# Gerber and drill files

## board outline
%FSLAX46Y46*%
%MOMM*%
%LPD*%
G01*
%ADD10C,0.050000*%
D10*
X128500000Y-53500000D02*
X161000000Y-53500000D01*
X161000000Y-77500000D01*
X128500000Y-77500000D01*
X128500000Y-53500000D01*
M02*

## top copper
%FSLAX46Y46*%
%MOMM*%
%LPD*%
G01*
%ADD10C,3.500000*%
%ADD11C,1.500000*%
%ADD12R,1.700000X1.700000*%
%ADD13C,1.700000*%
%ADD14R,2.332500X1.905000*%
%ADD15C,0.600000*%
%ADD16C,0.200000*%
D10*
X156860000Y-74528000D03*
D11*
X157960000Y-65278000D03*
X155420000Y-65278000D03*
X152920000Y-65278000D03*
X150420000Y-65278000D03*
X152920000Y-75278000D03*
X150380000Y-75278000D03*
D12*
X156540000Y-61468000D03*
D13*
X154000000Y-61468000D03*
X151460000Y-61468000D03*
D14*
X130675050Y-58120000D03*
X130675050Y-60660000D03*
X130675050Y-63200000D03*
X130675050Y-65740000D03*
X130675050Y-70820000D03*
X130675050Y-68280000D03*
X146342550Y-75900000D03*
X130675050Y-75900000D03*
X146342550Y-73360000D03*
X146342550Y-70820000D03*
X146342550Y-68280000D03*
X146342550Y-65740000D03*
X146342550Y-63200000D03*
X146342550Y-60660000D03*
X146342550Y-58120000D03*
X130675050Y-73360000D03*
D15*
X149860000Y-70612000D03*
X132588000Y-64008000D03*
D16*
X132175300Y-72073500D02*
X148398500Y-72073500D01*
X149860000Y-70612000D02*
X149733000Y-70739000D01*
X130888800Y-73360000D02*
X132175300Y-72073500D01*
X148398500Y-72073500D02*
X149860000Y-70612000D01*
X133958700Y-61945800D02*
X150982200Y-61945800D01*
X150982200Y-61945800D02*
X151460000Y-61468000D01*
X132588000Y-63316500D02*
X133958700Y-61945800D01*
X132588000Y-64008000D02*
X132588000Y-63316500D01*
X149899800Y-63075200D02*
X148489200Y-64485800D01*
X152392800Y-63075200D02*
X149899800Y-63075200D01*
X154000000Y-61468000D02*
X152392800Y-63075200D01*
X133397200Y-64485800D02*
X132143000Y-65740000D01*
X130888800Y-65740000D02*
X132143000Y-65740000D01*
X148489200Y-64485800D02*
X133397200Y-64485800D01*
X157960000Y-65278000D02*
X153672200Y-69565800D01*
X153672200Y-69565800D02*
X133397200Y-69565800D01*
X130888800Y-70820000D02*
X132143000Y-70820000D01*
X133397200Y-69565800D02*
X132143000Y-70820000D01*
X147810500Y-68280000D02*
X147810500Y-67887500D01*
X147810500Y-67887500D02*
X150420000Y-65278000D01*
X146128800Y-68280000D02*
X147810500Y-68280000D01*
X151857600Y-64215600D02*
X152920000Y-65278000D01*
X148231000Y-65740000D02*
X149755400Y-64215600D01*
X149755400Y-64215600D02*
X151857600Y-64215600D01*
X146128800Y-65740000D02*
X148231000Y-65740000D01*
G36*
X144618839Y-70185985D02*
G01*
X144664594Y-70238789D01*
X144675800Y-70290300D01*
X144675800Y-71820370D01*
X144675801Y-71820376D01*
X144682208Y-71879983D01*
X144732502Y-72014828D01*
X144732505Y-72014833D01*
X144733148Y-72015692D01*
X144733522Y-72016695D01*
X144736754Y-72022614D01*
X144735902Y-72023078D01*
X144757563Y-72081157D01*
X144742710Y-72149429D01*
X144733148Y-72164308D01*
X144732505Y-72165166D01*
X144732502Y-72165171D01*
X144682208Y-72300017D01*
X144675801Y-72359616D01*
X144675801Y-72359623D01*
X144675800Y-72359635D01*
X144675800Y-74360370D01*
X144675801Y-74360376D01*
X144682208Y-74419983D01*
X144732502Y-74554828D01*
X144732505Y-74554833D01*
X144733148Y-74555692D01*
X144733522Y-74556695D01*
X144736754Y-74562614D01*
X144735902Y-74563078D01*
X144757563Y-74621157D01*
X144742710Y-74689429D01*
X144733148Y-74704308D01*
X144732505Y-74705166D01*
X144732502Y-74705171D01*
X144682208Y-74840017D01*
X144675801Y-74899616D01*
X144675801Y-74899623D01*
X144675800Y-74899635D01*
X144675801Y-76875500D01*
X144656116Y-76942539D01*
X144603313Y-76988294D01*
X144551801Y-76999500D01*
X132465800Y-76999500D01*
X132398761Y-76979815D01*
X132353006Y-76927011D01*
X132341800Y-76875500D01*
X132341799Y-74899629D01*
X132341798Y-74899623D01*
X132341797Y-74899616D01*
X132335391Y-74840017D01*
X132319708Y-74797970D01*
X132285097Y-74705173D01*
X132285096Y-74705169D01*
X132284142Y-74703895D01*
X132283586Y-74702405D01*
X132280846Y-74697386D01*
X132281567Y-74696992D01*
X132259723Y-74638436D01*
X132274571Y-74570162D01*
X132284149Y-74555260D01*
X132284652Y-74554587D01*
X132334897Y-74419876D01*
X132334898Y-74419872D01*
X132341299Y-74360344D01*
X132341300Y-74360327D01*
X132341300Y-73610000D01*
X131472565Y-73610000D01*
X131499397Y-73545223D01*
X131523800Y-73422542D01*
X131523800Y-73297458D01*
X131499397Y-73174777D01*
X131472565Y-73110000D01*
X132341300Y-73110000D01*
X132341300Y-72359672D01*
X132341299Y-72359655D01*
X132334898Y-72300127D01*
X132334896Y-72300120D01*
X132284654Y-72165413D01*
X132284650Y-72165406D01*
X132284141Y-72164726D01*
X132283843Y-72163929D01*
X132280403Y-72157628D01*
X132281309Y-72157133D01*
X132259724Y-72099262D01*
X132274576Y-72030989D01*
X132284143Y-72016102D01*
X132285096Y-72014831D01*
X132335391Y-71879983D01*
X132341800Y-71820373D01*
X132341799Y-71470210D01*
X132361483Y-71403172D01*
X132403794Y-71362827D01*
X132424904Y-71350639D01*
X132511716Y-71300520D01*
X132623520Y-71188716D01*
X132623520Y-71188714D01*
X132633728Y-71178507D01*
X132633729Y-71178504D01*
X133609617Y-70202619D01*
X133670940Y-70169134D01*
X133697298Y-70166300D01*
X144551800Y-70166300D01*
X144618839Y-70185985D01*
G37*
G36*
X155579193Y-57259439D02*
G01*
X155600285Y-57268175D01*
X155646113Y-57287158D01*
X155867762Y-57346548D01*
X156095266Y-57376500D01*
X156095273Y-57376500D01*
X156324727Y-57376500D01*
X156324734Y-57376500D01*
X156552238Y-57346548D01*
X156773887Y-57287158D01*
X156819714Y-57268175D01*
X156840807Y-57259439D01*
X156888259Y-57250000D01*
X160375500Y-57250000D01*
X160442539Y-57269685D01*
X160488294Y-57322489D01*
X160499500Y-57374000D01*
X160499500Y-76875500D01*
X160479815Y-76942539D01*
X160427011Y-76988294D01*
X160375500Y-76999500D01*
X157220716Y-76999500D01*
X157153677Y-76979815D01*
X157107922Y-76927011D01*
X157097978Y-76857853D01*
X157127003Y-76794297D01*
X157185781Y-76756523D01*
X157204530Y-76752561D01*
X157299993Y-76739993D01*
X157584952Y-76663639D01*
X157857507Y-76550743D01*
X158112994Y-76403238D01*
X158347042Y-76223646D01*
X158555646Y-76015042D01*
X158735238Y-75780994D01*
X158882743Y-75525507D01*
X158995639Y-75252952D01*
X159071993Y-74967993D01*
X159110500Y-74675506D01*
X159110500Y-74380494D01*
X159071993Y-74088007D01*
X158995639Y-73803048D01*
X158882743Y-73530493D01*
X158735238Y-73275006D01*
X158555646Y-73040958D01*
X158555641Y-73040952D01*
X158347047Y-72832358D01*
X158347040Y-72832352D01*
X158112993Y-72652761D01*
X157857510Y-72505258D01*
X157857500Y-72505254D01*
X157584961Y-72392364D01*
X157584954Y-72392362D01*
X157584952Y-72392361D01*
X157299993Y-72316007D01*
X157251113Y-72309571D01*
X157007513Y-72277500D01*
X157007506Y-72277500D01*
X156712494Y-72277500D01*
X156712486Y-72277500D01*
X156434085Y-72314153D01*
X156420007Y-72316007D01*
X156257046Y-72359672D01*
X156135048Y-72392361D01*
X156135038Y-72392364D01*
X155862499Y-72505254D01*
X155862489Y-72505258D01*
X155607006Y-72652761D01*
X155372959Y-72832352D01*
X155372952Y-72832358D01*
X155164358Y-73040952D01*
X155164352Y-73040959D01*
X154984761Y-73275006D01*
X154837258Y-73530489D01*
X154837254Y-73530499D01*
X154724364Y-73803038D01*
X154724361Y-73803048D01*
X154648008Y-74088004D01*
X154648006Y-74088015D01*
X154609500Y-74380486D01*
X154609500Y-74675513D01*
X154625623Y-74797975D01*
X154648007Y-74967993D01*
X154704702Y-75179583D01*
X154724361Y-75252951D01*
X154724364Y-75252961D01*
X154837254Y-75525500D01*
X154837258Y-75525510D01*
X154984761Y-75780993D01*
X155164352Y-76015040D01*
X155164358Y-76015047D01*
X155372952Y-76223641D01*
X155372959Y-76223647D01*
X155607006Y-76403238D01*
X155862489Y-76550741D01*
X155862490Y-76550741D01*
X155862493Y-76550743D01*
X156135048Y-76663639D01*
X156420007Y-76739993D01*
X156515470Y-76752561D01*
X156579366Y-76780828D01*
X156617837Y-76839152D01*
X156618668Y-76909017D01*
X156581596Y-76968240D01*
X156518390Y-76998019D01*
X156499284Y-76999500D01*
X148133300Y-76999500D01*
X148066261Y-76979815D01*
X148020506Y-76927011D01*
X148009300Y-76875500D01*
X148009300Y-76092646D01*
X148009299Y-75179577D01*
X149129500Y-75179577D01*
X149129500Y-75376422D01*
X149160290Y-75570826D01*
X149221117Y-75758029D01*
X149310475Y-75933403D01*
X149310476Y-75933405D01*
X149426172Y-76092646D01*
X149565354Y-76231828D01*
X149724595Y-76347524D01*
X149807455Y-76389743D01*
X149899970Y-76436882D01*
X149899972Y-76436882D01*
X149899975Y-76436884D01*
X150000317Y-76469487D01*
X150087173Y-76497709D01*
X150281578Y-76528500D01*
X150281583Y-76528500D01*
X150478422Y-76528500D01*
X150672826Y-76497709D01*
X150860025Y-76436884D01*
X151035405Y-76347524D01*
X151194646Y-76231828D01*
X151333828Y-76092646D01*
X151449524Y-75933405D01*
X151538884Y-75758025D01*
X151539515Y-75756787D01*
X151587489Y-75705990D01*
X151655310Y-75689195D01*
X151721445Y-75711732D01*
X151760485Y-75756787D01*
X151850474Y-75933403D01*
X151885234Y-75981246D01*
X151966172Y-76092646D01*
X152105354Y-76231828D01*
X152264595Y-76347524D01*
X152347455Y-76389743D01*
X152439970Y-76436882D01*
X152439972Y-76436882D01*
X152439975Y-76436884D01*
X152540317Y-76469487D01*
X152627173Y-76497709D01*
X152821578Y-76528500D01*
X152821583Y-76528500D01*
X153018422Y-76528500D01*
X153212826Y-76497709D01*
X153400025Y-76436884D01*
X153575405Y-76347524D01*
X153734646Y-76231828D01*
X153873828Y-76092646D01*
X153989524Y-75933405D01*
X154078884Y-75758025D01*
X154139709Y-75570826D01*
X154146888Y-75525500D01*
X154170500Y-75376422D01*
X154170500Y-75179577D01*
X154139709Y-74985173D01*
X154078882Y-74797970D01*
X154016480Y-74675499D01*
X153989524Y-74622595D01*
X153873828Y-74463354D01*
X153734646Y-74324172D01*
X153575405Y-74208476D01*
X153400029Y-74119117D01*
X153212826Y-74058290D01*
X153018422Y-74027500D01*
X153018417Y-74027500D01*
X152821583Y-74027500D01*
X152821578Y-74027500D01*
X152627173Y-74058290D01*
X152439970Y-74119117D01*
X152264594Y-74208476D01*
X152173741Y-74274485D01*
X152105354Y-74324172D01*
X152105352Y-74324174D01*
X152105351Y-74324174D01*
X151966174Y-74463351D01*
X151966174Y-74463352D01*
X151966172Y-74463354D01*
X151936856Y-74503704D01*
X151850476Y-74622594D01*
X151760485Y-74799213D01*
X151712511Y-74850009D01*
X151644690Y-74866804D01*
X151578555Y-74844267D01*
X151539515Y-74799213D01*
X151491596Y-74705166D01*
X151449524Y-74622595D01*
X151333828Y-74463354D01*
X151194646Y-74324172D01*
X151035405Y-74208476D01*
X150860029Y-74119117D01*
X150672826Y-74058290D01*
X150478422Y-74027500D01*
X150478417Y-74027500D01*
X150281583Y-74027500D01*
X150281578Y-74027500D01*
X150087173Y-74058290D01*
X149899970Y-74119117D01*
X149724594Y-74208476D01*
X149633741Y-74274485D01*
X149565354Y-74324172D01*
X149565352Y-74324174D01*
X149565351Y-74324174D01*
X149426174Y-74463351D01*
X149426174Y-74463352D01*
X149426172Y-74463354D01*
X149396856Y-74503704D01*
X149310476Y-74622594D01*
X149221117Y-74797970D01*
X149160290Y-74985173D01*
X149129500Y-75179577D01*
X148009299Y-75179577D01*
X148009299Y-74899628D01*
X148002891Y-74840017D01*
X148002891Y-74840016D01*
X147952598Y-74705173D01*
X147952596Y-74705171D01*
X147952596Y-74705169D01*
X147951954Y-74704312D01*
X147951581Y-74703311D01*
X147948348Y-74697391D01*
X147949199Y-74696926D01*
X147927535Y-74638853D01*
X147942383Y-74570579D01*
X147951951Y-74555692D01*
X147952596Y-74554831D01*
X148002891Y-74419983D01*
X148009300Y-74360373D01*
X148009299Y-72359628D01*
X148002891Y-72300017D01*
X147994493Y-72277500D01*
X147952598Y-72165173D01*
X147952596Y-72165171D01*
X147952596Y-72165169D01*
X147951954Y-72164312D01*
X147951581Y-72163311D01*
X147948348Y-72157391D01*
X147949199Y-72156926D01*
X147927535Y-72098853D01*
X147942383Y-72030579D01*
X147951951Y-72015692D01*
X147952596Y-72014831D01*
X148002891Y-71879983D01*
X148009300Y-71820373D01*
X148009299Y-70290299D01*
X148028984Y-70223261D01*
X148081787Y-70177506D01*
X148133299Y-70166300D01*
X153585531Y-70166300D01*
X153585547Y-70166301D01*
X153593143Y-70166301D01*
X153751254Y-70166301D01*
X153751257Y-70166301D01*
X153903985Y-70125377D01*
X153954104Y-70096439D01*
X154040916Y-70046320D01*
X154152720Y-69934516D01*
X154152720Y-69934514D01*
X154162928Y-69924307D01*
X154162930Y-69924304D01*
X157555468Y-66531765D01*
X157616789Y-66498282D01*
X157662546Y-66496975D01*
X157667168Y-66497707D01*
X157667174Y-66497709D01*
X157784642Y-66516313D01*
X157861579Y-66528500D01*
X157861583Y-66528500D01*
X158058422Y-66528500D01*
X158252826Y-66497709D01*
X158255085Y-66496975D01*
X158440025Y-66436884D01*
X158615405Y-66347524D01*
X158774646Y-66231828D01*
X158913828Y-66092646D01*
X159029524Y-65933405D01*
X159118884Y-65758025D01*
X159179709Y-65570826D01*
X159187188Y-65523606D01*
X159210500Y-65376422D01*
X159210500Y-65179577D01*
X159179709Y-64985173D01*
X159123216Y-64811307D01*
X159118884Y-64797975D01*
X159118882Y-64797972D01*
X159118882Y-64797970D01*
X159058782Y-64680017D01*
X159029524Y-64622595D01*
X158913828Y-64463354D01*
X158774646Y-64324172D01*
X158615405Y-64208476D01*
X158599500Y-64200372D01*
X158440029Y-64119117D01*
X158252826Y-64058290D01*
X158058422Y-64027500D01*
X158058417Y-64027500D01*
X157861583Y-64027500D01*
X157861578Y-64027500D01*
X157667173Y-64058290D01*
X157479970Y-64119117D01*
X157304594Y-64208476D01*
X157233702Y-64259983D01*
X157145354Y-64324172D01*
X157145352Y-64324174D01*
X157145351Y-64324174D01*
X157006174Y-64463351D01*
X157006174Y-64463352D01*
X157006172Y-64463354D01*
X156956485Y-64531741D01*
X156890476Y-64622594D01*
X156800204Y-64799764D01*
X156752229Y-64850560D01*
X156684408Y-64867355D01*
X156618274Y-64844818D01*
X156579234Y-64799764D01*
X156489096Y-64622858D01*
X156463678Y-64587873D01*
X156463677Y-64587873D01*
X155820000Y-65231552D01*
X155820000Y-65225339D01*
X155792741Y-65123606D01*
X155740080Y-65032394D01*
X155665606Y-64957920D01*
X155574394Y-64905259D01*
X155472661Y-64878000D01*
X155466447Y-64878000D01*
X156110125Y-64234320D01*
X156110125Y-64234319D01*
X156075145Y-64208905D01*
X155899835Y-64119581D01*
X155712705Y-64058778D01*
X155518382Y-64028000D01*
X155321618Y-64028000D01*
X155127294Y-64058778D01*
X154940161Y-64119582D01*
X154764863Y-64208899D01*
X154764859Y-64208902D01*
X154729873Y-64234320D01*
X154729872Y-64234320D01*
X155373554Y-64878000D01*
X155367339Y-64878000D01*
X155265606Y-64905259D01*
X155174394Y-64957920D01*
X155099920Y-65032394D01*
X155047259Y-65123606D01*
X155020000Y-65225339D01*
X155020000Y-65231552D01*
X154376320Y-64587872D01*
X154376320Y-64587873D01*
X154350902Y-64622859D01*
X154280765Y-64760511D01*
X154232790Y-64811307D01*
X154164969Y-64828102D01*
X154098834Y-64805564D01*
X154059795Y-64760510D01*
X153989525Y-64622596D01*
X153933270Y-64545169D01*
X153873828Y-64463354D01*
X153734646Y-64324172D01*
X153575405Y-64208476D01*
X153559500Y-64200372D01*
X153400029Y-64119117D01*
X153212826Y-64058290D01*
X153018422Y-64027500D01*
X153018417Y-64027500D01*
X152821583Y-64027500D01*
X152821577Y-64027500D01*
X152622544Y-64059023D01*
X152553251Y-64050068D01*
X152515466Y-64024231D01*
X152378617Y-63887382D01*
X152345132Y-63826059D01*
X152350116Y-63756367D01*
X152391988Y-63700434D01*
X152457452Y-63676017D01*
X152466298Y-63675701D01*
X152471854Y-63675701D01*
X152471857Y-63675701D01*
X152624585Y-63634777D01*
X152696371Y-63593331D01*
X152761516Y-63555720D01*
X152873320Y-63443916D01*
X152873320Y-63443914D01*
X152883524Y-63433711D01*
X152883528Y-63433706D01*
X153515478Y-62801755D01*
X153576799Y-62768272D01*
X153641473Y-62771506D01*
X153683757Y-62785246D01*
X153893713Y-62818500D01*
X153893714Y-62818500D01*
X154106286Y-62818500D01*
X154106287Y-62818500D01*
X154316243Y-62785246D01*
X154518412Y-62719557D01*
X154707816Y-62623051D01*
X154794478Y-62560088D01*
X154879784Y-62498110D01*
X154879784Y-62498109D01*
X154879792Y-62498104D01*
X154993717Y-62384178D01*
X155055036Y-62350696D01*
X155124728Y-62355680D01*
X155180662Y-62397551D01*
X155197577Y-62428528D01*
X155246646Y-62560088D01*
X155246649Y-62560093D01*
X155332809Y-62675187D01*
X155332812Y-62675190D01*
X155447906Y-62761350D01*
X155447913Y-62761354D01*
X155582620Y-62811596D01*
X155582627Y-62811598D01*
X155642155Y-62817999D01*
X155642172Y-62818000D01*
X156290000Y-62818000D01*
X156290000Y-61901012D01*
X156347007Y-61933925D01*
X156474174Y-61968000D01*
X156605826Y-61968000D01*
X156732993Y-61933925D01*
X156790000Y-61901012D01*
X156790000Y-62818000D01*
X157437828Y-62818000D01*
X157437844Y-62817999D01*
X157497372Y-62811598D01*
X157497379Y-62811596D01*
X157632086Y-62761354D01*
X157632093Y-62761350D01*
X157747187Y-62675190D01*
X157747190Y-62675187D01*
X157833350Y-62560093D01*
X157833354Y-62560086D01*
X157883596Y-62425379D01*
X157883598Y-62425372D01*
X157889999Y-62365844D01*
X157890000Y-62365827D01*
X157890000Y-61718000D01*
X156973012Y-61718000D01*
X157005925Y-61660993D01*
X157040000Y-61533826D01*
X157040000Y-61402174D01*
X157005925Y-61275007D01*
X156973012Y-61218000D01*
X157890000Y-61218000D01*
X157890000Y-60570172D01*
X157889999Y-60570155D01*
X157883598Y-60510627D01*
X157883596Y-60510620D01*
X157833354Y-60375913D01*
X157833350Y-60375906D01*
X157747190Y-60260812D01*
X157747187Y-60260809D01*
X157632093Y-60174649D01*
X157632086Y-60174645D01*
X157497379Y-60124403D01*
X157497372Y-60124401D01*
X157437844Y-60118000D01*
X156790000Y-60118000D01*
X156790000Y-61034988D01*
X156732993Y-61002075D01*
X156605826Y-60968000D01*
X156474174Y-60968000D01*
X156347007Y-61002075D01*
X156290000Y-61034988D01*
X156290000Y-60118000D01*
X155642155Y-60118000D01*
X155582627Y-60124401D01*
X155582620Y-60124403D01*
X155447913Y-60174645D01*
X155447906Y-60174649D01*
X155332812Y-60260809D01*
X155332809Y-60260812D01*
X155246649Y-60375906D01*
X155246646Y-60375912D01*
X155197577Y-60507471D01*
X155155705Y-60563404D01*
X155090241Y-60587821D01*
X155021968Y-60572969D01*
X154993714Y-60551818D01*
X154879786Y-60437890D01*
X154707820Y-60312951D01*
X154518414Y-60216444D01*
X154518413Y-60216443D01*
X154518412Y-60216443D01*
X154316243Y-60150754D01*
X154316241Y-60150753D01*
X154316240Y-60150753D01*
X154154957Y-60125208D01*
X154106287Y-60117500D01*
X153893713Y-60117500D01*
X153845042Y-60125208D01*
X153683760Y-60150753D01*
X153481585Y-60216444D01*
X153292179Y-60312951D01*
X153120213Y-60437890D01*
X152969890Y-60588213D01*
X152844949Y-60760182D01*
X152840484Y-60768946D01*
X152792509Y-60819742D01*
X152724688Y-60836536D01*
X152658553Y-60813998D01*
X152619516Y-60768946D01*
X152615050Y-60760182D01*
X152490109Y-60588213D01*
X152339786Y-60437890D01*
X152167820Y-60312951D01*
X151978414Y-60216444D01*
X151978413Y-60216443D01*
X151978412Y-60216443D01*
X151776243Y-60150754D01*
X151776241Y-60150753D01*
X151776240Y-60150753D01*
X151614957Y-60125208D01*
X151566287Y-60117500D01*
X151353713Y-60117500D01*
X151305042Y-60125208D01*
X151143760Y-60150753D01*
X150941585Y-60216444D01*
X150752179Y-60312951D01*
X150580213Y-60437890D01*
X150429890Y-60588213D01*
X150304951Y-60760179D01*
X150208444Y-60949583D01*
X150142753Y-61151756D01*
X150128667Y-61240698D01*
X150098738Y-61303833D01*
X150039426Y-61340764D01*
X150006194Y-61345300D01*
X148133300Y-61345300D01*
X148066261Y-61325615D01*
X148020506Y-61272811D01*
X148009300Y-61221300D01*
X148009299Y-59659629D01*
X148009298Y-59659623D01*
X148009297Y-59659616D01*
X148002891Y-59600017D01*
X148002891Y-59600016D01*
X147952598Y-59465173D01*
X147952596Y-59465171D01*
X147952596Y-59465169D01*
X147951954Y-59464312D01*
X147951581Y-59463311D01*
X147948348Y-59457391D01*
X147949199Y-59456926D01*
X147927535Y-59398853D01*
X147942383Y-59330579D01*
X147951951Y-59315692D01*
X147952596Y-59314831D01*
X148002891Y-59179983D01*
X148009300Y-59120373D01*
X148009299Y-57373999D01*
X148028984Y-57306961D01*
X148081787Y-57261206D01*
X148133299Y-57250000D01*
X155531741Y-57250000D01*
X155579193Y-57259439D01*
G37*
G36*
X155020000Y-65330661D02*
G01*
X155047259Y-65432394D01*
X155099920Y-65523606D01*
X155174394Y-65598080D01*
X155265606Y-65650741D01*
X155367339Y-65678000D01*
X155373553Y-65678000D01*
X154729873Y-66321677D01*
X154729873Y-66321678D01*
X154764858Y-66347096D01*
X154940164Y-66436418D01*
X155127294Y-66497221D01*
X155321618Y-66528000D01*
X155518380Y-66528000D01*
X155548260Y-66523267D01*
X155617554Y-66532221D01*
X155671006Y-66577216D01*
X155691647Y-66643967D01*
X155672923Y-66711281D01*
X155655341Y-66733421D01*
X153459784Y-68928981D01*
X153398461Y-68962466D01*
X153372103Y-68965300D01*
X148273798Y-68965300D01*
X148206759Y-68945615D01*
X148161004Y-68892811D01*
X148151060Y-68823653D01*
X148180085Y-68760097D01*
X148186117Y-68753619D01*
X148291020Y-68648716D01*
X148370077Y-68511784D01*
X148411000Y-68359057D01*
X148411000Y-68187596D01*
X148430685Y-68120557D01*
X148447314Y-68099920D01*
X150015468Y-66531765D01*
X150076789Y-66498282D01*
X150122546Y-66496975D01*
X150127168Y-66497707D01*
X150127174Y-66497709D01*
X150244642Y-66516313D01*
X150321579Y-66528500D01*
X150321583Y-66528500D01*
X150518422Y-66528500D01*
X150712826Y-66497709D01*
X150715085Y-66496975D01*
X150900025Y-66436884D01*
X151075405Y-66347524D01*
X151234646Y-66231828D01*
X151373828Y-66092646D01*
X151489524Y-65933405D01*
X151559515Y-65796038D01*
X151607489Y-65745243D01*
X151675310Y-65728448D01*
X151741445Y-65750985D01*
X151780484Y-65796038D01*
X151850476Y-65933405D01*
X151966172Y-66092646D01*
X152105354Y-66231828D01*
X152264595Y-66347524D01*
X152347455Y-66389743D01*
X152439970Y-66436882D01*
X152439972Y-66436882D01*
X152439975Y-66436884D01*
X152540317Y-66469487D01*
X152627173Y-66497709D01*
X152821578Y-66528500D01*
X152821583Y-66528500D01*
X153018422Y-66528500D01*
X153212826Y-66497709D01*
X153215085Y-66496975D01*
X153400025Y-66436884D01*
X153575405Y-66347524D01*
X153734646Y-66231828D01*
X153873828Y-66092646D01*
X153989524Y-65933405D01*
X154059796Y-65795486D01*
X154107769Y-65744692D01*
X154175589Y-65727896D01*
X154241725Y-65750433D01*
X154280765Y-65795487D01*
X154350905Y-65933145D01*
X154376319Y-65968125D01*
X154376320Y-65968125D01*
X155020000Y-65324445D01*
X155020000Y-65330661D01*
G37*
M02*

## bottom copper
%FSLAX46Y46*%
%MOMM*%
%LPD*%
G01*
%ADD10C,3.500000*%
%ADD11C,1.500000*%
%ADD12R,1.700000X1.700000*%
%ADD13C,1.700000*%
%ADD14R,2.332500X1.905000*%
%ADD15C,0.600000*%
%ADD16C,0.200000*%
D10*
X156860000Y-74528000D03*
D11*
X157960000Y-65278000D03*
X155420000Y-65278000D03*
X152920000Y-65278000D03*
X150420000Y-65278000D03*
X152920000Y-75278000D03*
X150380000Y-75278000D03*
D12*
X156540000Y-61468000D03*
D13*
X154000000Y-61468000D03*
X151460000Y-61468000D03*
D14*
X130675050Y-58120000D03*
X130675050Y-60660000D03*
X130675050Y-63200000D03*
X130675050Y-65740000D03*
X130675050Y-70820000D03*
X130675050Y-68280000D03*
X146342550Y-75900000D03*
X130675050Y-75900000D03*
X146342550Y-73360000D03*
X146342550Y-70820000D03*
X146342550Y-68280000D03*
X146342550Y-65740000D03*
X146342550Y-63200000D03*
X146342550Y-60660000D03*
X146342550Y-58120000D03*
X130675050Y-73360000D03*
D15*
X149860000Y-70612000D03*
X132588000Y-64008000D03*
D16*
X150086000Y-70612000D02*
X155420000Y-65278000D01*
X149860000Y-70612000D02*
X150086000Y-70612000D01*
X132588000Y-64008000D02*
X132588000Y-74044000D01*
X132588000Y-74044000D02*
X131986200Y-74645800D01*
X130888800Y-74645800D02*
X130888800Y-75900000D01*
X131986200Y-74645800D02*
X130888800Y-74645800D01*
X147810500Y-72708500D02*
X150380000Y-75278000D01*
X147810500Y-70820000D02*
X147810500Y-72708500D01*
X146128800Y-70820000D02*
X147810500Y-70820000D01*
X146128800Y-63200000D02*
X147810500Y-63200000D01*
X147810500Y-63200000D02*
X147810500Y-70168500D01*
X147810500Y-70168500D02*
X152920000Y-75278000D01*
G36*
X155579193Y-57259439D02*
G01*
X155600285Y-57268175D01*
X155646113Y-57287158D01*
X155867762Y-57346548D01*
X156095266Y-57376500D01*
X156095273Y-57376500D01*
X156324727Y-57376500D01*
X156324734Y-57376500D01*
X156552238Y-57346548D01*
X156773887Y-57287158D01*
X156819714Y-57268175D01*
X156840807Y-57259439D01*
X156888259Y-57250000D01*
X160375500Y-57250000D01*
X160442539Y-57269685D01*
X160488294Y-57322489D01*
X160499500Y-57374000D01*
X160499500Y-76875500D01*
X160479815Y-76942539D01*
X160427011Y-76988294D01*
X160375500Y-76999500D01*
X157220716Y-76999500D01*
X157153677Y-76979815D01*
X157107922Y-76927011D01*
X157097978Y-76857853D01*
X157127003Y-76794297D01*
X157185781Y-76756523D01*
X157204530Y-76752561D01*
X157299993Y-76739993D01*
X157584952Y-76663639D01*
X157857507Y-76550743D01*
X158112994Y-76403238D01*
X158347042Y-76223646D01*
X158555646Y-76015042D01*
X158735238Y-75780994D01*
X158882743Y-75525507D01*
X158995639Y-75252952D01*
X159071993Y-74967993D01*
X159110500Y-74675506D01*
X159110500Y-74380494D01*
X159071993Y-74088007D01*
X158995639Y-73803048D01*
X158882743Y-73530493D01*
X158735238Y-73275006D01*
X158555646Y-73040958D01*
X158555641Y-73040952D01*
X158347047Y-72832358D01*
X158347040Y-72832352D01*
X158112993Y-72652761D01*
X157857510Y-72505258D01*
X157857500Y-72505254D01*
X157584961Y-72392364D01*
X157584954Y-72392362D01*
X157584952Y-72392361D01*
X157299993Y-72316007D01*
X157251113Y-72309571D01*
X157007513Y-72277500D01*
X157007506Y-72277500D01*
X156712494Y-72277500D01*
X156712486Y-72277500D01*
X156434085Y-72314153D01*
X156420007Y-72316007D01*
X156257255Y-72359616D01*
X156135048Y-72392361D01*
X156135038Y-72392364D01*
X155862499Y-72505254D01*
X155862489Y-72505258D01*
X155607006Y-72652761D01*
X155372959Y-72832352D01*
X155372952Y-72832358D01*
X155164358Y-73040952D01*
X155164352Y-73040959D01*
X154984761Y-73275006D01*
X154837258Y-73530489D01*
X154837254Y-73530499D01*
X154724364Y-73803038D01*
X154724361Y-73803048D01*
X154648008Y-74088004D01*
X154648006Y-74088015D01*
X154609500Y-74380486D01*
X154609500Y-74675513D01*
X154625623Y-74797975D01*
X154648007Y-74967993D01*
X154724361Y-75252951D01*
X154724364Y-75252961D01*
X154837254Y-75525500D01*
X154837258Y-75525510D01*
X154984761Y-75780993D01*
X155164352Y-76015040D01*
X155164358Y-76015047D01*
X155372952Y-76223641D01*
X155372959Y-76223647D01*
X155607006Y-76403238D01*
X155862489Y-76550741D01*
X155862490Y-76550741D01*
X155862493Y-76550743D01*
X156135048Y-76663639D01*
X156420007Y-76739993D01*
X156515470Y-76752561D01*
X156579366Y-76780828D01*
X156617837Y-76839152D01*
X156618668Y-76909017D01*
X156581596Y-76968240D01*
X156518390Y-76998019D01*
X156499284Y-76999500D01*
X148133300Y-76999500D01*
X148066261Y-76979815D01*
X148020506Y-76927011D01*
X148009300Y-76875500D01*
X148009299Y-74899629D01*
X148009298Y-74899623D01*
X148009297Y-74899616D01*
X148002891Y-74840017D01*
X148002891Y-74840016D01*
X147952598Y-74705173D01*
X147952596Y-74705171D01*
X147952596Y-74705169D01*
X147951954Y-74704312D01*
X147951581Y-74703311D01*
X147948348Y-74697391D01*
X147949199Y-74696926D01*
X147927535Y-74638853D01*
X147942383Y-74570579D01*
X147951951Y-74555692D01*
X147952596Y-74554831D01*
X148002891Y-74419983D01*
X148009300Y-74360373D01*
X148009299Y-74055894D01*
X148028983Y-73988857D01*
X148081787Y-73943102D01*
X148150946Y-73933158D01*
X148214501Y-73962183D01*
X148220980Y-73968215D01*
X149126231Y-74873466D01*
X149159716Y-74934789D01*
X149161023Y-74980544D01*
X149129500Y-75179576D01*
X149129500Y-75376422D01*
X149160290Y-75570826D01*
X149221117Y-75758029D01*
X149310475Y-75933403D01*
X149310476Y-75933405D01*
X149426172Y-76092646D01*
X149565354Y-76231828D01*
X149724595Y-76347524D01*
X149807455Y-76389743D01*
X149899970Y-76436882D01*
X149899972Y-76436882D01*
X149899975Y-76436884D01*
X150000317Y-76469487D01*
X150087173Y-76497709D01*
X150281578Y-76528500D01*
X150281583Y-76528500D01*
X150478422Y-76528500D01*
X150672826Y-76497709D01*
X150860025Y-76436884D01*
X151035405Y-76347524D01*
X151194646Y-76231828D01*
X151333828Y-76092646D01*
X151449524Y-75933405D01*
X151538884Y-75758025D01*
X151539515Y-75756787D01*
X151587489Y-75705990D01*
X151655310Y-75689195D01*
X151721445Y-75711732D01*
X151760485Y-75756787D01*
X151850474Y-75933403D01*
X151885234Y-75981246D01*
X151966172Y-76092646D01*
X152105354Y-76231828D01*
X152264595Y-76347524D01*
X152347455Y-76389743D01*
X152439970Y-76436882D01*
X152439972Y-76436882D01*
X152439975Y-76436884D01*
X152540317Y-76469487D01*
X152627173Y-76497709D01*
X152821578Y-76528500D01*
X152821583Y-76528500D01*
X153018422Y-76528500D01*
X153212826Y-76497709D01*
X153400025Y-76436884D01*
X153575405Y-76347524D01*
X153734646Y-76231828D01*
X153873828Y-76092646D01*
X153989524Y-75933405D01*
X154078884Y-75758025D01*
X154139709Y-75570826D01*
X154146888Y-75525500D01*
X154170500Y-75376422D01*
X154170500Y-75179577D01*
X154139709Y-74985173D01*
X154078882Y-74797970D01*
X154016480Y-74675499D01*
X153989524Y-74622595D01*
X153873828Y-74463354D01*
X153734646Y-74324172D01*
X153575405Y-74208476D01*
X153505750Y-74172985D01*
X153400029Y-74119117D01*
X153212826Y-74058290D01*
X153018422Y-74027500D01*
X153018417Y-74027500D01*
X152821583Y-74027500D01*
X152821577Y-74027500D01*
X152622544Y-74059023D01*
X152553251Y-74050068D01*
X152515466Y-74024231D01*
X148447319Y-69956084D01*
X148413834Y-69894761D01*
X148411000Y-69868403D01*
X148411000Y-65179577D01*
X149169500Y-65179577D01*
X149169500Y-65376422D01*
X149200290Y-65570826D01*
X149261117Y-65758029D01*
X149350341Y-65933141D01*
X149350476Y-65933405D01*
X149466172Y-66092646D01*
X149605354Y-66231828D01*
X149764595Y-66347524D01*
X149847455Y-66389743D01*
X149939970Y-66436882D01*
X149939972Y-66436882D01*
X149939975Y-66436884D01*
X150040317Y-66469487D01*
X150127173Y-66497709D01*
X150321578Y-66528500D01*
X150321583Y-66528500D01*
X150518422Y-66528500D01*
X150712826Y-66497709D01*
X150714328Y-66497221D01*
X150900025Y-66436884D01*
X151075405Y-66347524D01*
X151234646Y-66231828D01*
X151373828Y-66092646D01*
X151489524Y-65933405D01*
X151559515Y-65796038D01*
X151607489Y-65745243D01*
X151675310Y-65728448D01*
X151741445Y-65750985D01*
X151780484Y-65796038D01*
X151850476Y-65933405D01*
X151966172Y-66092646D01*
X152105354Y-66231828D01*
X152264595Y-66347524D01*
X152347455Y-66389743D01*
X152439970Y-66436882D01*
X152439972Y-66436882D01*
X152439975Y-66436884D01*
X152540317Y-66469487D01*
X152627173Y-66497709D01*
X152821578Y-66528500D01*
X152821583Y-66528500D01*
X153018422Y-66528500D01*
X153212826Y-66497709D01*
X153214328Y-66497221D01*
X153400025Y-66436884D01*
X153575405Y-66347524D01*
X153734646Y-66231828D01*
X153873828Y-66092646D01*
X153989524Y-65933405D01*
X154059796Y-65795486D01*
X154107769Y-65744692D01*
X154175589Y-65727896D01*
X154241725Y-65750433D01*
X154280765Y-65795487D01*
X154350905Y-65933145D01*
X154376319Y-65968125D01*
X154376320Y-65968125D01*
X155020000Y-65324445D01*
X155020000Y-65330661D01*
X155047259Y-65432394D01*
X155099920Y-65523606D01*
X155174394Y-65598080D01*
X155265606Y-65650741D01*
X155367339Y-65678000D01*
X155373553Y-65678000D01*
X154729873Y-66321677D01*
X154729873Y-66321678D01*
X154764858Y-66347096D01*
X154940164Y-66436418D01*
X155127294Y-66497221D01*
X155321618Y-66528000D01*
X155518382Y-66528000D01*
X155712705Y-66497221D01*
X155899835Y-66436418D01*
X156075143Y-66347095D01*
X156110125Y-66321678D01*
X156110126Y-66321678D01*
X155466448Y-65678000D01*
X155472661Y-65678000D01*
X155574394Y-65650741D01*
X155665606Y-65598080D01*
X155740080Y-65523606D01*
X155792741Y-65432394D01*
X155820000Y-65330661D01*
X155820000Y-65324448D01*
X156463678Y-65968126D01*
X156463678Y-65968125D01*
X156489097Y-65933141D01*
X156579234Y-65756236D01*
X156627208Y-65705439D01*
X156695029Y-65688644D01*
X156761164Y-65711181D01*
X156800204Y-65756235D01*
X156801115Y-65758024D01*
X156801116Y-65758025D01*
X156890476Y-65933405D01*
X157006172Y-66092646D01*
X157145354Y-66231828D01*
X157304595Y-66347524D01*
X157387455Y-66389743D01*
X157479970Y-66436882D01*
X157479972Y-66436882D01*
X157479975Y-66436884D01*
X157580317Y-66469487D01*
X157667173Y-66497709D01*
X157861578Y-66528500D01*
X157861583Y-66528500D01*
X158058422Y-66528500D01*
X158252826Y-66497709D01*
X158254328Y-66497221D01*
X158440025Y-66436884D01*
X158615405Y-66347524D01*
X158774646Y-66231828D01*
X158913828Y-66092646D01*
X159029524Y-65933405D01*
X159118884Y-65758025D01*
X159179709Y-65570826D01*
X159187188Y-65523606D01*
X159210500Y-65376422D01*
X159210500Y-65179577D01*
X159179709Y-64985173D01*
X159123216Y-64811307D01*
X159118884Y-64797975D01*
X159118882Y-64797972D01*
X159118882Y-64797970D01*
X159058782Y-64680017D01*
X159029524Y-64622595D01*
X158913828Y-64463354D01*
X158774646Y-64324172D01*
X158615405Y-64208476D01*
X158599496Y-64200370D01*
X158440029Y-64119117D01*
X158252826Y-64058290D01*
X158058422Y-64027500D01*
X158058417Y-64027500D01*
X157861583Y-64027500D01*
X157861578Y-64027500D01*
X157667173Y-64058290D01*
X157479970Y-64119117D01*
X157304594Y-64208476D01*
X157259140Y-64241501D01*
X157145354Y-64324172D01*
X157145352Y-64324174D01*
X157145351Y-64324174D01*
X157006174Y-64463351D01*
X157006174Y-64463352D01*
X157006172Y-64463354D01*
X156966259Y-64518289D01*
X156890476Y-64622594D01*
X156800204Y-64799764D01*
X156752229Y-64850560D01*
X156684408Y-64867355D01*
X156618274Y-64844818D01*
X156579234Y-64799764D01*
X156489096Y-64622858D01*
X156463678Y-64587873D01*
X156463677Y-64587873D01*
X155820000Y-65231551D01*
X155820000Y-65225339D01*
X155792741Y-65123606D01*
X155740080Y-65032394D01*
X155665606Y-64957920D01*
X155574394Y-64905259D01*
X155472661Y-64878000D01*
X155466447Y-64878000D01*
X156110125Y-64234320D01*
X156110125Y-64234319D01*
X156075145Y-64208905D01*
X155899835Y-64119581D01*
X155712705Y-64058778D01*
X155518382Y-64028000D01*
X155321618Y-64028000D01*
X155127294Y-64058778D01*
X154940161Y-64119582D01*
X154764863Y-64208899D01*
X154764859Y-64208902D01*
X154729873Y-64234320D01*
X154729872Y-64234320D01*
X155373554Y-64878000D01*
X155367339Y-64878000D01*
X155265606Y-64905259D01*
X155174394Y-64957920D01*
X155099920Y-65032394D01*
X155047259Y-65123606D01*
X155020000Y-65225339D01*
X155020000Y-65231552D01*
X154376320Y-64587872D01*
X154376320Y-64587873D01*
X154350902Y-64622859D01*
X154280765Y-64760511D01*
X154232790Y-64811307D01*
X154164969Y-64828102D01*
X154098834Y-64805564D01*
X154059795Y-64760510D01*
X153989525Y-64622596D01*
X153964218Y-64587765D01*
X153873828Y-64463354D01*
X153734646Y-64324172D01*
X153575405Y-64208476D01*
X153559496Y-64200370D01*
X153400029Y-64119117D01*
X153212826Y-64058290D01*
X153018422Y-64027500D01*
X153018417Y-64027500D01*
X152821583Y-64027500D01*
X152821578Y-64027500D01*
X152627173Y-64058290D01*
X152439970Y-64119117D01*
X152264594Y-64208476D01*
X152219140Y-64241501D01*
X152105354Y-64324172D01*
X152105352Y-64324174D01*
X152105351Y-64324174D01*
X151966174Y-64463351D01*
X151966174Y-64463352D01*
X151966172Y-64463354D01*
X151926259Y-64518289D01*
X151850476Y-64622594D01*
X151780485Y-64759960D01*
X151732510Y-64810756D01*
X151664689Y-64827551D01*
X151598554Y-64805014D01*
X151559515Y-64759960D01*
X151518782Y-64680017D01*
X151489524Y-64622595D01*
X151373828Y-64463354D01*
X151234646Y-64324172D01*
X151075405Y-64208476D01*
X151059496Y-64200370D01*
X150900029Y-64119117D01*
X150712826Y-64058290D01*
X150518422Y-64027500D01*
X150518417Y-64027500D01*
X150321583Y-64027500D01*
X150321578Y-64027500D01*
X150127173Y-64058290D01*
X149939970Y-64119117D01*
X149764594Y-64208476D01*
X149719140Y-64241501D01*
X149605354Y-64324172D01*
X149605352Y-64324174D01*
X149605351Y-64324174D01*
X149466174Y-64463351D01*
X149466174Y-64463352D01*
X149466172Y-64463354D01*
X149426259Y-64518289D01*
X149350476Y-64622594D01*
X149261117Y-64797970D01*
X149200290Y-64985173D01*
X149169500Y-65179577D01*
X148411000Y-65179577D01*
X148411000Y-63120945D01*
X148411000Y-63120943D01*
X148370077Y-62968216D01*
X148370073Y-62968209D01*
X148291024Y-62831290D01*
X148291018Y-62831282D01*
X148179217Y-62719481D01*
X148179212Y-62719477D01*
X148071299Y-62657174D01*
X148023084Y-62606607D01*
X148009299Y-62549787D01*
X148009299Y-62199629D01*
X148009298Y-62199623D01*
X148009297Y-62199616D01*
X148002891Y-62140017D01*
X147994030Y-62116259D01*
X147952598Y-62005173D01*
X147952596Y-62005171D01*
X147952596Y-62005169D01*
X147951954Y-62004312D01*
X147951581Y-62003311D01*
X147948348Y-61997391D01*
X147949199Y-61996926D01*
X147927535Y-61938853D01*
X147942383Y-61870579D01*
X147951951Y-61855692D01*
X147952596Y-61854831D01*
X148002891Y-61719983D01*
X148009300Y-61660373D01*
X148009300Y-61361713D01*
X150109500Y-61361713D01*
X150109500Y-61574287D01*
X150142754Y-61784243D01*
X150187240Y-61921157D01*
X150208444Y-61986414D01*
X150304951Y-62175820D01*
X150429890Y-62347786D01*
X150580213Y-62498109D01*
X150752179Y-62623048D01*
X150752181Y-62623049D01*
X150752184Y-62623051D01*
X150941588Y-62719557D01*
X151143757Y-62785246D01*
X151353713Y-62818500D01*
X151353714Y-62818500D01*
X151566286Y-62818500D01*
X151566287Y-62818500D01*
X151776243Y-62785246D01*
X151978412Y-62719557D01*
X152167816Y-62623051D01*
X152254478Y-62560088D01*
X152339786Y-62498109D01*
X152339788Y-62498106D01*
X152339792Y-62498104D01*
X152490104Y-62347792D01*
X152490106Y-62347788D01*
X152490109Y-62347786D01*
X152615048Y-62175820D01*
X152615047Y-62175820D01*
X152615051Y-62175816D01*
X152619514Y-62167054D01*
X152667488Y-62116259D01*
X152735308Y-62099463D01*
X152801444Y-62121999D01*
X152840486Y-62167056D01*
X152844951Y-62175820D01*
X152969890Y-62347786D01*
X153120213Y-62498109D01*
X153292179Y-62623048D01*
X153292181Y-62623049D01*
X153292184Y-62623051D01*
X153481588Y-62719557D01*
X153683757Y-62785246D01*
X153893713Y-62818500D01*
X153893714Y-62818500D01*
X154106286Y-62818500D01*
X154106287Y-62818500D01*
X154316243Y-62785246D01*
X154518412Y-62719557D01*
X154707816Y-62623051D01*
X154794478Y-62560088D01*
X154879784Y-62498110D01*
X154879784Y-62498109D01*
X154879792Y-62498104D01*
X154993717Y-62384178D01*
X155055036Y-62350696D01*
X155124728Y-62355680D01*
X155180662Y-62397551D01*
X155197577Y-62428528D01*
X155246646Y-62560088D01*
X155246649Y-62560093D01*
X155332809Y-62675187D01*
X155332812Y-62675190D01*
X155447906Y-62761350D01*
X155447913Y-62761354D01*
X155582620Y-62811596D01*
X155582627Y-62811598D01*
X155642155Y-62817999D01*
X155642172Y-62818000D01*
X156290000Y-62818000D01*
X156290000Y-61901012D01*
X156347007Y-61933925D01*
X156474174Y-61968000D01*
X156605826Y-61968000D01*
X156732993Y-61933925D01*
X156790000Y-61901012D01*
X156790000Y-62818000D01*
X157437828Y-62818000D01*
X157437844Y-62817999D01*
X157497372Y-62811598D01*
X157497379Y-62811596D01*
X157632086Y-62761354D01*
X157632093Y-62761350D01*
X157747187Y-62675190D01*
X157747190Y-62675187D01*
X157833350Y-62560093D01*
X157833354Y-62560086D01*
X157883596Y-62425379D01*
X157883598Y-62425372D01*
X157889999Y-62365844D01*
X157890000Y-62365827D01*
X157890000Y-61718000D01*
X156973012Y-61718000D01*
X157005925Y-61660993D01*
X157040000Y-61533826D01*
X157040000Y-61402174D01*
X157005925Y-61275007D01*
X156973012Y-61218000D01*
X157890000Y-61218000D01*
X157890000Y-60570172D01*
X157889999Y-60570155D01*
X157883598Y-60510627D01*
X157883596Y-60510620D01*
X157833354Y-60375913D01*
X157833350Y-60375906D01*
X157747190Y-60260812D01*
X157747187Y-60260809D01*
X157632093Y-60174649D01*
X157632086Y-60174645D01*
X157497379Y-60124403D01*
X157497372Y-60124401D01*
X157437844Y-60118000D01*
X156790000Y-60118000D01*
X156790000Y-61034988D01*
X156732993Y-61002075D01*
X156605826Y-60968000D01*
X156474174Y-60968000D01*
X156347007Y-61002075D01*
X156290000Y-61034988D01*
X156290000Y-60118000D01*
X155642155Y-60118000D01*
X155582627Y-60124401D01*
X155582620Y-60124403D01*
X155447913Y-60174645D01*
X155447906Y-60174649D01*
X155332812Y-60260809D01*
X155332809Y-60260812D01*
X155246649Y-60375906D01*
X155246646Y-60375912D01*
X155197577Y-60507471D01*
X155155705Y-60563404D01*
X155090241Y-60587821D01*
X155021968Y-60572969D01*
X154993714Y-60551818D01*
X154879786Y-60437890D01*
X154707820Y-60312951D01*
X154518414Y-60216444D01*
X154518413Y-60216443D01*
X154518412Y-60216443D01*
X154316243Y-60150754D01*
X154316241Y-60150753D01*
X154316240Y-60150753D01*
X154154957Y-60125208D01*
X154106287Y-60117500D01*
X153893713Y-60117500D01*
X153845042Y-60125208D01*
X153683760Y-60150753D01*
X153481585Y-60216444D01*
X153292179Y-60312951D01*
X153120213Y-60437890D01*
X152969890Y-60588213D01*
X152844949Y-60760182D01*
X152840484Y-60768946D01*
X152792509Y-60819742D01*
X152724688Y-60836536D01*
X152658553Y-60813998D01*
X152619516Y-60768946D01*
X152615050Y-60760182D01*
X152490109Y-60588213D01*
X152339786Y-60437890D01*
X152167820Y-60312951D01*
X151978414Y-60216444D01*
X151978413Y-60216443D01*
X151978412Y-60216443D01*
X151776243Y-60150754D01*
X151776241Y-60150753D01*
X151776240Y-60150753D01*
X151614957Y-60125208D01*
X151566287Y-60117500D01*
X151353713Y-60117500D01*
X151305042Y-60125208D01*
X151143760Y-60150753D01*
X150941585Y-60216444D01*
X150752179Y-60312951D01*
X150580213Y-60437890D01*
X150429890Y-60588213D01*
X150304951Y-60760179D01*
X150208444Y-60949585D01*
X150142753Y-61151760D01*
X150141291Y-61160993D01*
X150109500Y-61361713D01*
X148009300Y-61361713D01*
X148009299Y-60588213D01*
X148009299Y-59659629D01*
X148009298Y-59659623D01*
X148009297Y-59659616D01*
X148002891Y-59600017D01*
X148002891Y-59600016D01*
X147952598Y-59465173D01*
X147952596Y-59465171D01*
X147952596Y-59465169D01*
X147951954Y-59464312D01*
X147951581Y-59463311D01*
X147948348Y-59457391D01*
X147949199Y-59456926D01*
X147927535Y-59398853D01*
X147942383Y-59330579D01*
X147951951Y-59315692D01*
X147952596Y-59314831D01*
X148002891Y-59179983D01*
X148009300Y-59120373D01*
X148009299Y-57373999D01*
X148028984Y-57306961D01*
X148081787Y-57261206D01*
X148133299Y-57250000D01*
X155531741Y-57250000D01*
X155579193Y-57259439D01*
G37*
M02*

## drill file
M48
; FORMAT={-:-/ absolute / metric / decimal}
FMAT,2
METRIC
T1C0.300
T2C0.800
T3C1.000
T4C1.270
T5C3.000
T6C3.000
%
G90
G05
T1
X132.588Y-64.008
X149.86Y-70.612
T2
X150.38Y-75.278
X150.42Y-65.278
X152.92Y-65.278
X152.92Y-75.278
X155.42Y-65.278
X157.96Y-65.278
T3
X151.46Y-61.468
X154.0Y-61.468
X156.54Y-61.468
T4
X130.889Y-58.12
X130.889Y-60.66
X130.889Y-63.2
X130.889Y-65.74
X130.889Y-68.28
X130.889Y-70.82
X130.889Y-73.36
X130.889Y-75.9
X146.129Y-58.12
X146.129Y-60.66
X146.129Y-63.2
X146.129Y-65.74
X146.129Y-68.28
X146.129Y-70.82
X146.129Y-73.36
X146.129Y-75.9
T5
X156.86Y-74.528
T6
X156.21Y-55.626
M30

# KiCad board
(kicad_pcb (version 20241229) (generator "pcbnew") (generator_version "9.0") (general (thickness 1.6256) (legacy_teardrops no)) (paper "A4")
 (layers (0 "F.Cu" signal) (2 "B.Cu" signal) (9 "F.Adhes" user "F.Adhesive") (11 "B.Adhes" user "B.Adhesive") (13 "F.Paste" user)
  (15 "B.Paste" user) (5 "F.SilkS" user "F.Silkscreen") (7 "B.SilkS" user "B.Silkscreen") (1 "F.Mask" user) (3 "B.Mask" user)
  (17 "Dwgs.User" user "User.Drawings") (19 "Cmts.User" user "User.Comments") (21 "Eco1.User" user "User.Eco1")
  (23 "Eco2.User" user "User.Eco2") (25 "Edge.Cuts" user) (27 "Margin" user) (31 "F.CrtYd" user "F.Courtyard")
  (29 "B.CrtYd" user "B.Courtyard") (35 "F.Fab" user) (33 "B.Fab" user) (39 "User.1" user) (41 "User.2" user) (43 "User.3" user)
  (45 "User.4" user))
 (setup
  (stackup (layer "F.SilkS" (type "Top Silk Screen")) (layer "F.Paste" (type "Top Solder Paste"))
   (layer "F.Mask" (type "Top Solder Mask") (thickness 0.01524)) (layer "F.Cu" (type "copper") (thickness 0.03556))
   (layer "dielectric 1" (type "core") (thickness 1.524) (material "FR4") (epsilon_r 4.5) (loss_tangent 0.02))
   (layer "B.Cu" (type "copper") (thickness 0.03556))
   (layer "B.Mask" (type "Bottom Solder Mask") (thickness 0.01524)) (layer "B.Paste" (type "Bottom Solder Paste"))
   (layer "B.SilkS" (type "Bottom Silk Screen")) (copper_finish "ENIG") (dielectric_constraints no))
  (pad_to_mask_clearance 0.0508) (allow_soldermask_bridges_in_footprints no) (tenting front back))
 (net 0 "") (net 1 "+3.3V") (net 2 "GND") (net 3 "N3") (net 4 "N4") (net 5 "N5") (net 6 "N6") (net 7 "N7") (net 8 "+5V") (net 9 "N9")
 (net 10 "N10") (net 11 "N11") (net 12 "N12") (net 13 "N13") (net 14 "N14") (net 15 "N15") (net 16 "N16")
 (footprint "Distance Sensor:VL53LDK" (layer "F.Cu") (at 154.21 70.278 -90)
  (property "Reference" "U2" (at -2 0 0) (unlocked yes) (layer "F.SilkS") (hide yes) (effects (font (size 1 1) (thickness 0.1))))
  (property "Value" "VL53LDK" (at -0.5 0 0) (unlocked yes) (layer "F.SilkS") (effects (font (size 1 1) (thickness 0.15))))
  (pad "" thru_hole circle (at 4.25 -2.65 270) (size 3.5 3.5) (drill 3) (layers "*.Cu" "*.Mask") (remove_unused_layers no))
  (pad "1" thru_hole circle (at -5 -3.75 270) (size 1.5 1.5) (drill 0.8) (layers "*.Cu" "*.Mask") (remove_unused_layers no) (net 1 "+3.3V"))
  (pad "2" thru_hole circle (at -5 -1.21 270) (size 1.5 1.5) (drill 0.8) (layers "*.Cu" "*.Mask") (remove_unused_layers no) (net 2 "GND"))
  (pad "3" thru_hole circle (at -5 1.29 270) (size 1.5 1.5) (drill 0.8) (layers "*.Cu" "*.Mask") (remove_unused_layers no) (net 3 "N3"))
  (pad "4" thru_hole circle (at -5 3.79 270) (size 1.5 1.5) (drill 0.8) (layers "*.Cu" "*.Mask") (remove_unused_layers no) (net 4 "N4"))
  (pad "5" thru_hole circle (at 5 1.29 270) (size 1.5 1.5) (drill 0.8) (layers "*.Cu" "*.Mask") (remove_unused_layers no) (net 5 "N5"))
  (pad "6" thru_hole circle (at 5 3.83 270) (size 1.5 1.5) (drill 0.8) (layers "*.Cu" "*.Mask") (remove_unused_layers no) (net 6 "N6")))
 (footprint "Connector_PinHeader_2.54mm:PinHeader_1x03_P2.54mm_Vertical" (layer "F.Cu") (at 156.54 61.468 -90)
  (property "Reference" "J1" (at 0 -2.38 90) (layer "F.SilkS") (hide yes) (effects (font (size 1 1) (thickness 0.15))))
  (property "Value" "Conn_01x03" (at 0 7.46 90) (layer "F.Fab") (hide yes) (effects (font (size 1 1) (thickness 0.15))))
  (pad "1" thru_hole rect (at 0 0 270) (size 1.7 1.7) (drill 1) (layers "*.Cu" "*.Mask") (remove_unused_layers no) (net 2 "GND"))
  (pad "2" thru_hole circle (at 0 2.54 270) (size 1.7 1.7) (drill 1) (layers "*.Cu" "*.Mask") (remove_unused_layers no) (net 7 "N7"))
  (pad "3" thru_hole circle (at 0 5.08 270) (size 1.7 1.7) (drill 1) (layers "*.Cu" "*.Mask") (remove_unused_layers no) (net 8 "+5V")))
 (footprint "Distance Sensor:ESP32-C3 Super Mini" (layer "F.Cu") (at 138.5088 66 180)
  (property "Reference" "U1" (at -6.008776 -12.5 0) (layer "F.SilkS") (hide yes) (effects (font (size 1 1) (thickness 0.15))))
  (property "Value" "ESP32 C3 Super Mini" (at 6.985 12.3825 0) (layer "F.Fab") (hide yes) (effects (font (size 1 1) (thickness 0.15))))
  (pad "0" thru_hole rect (at 7.62 7.88 180) (size 2.3325 1.905) (drill 1.27 (offset 0.21375 0)) (layers "*.Cu" "*.Mask")
   (remove_unused_layers no) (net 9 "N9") (solder_mask_margin 0.102))
  (pad "1" thru_hole rect (at 7.62 5.34 180) (size 2.3325 1.905) (drill 1.27 (offset 0.21375 0)) (layers "*.Cu" "*.Mask")
   (remove_unused_layers no) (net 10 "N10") (solder_mask_margin 0.102))
  (pad "2" thru_hole rect (at 7.62 2.8 180) (size 2.3325 1.905) (drill 1.27 (offset 0.21375 0)) (layers "*.Cu" "*.Mask")
   (remove_unused_layers no) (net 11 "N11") (solder_mask_margin 0.102))
  (pad "3" thru_hole rect (at 7.62 0.26 180) (size 2.3325 1.905) (drill 1.27 (offset 0.21375 0)) (layers "*.Cu" "*.Mask")
   (remove_unused_layers no) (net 7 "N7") (solder_mask_margin 0.102))
  (pad "3.3" thru_hole rect (at 7.62 -4.82 180) (size 2.3325 1.905) (drill 1.27 (offset 0.21375 0)) (layers "*.Cu" "*.Mask")
   (remove_unused_layers no) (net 1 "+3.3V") (solder_mask_margin 0.102))
  (pad "4" thru_hole rect (at 7.62 -2.28 180) (size 2.3325 1.905) (drill 1.27 (offset 0.21375 0)) (layers "*.Cu" "*.Mask")
   (remove_unused_layers no) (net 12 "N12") (solder_mask_margin 0.102))
  (pad "5" thru_hole rect (at -7.62 -9.9 180) (size 2.3325 1.905) (drill 1.27 (offset -0.21375 0)) (layers "*.Cu" "*.Mask")
   (remove_unused_layers no) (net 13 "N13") (solder_mask_margin 0.102))
  (pad "5V" thru_hole rect (at 7.62 -9.9 180) (size 2.3325 1.905) (drill 1.27 (offset 0.21375 0)) (layers "*.Cu" "*.Mask")
   (remove_unused_layers no) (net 8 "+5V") (solder_mask_margin 0.102))
  (pad "6" thru_hole rect (at -7.62 -7.36 180) (size 2.3325 1.905) (drill 1.27 (offset -0.21375 0)) (layers "*.Cu" "*.Mask")
   (remove_unused_layers no) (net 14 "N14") (solder_mask_margin 0.102))
  (pad "7" thru_hole rect (at -7.62 -4.82 180) (size 2.3325 1.905) (drill 1.27 (offset -0.21375 0)) (layers "*.Cu" "*.Mask")
   (remove_unused_layers no) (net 6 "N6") (solder_mask_margin 0.102))
  (pad "8" thru_hole rect (at -7.62 -2.28 180) (size 2.3325 1.905) (drill 1.27 (offset -0.21375 0)) (layers "*.Cu" "*.Mask")
   (remove_unused_layers no) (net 4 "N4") (solder_mask_margin 0.102))
  (pad "9" thru_hole rect (at -7.62 0.26 180) (size 2.3325 1.905) (drill 1.27 (offset -0.21375 0)) (layers "*.Cu" "*.Mask")
   (remove_unused_layers no) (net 3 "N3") (solder_mask_margin 0.102))
  (pad "10" thru_hole rect (at -7.62 2.8 180) (size 2.3325 1.905) (drill 1.27 (offset -0.21375 0)) (layers "*.Cu" "*.Mask")
   (remove_unused_layers no) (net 5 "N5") (solder_mask_margin 0.102))
  (pad "20" thru_hole rect (at -7.62 5.34 180) (size 2.3325 1.905) (drill 1.27 (offset -0.21375 0)) (layers "*.Cu" "*.Mask")
   (remove_unused_layers no) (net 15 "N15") (solder_mask_margin 0.102))
  (pad "21" thru_hole rect (at -7.62 7.88 180) (size 2.3325 1.905) (drill 1.27 (offset -0.21375 0)) (layers "*.Cu" "*.Mask")
   (remove_unused_layers no) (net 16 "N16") (solder_mask_margin 0.102))
  (pad "G" thru_hole rect (at 7.62 -7.36 180) (size 2.3325 1.905) (drill 1.27 (offset 0.21375 0)) (layers "*.Cu" "*.Mask")
   (remove_unused_layers no) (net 2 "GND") (solder_mask_margin 0.102))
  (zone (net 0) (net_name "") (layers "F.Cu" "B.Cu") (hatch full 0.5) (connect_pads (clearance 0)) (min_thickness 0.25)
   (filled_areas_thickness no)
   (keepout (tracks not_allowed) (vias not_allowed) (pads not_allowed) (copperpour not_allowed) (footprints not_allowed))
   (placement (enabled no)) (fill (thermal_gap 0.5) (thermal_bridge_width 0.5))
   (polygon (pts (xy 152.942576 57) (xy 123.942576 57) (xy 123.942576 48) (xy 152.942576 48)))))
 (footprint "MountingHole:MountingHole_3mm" (layer "F.Cu") (at 156.21 55.626)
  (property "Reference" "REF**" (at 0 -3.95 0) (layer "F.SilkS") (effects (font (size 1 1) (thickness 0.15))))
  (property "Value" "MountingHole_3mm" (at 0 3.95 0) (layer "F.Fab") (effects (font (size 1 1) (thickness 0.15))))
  (pad "" np_thru_hole circle (at 0 0) (size 3 3) (drill 3) (layers "*.Cu" "*.Mask")))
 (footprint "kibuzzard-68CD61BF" (layer "B.Cu") (at 138.508776 65.532 -90)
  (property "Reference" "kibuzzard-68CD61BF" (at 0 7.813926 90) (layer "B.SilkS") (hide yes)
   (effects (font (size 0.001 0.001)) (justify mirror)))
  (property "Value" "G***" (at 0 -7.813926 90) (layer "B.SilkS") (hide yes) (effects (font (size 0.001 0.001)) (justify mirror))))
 (gr_rect (start 128.5 53.5) (end 161 77.5) (stroke (width 0.05) (type default)) (fill no) (layer "Edge.Cuts"))
 (segment (start 132.1753 72.0735) (end 148.3985 72.0735) (width 0.2) (layer "F.Cu") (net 2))
 (segment (start 149.86 70.612) (end 149.733 70.739) (width 0.2) (layer "F.Cu") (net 2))
 (segment (start 130.8888 73.36) (end 132.1753 72.0735) (width 0.2) (layer "F.Cu") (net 2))
 (segment (start 148.3985 72.0735) (end 149.86 70.612) (width 0.2) (layer "F.Cu") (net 2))
 (via (at 149.86 70.612) (size 0.6) (drill 0.3) (layers "F.Cu" "B.Cu") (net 2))
 (segment (start 150.086 70.612) (end 155.42 65.278) (width 0.2) (layer "B.Cu") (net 2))
 (segment (start 149.86 70.612) (end 150.086 70.612) (width 0.2) (layer "B.Cu") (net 2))
 (segment (start 133.9587 61.9458) (end 150.9822 61.9458) (width 0.2) (layer "F.Cu") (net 8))
 (segment (start 150.9822 61.9458) (end 151.46 61.468) (width 0.2) (layer "F.Cu") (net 8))
 (segment (start 132.588 63.3165) (end 133.9587 61.9458) (width 0.2) (layer "F.Cu") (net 8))
 (segment (start 132.588 64.008) (end 132.588 63.3165) (width 0.2) (layer "F.Cu") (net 8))
 (via (at 132.588 64.008) (size 0.6) (drill 0.3) (layers "F.Cu" "B.Cu") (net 8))
 (segment (start 132.588 64.008) (end 132.588 74.044) (width 0.2) (layer "B.Cu") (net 8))
 (segment (start 132.588 74.044) (end 131.9862 74.6458) (width 0.2) (layer "B.Cu") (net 8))
 (segment (start 130.8888 74.6458) (end 130.8888 75.9) (width 0.2) (layer "B.Cu") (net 8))
 (segment (start 131.9862 74.6458) (end 130.8888 74.6458) (width 0.2) (layer "B.Cu") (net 8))
 (segment (start 149.8998 63.0752) (end 148.4892 64.4858) (width 0.2) (layer "F.Cu") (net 7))
 (segment (start 152.3928 63.0752) (end 149.8998 63.0752) (width 0.2) (layer "F.Cu") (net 7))
 (segment (start 154 61.468) (end 152.3928 63.0752) (width 0.2) (layer "F.Cu") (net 7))
 (segment (start 133.3972 64.4858) (end 132.143 65.74) (width 0.2) (layer "F.Cu") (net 7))
 (segment (start 130.8888 65.74) (end 132.143 65.74) (width 0.2) (layer "F.Cu") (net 7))
 (segment (start 148.4892 64.4858) (end 133.3972 64.4858) (width 0.2) (layer "F.Cu") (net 7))
 (segment (start 157.96 65.278) (end 153.6722 69.5658) (width 0.2) (layer "F.Cu") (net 1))
 (segment (start 153.6722 69.5658) (end 133.3972 69.5658) (width 0.2) (layer "F.Cu") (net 1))
 (segment (start 130.8888 70.82) (end 132.143 70.82) (width 0.2) (layer "F.Cu") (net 1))
 (segment (start 133.3972 69.5658) (end 132.143 70.82) (width 0.2) (layer "F.Cu") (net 1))
 (segment (start 147.8105 72.7085) (end 150.38 75.278) (width 0.2) (layer "B.Cu") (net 6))
 (segment (start 147.8105 70.82) (end 147.8105 72.7085) (width 0.2) (layer "B.Cu") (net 6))
 (segment (start 146.1288 70.82) (end 147.8105 70.82) (width 0.2) (layer "B.Cu") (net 6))
 (segment (start 147.8105 68.28) (end 147.8105 67.8875) (width 0.2) (layer "F.Cu") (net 4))
 (segment (start 147.8105 67.8875) (end 150.42 65.278) (width 0.2) (layer "F.Cu") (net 4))
 (segment (start 146.1288 68.28) (end 147.8105 68.28) (width 0.2) (layer "F.Cu") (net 4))
 (segment (start 151.8576 64.2156) (end 152.92 65.278) (width 0.2) (layer "F.Cu") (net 3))
 (segment (start 148.231 65.74) (end 149.7554 64.2156) (width 0.2) (layer "F.Cu") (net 3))
 (segment (start 149.7554 64.2156) (end 151.8576 64.2156) (width 0.2) (layer "F.Cu") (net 3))
 (segment (start 146.1288 65.74) (end 148.231 65.74) (width 0.2) (layer "F.Cu") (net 3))
 (segment (start 146.1288 63.2) (end 147.8105 63.2) (width 0.2) (layer "B.Cu") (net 5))
 (segment (start 147.8105 63.2) (end 147.8105 70.1685) (width 0.2) (layer "B.Cu") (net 5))
 (segment (start 147.8105 70.1685) (end 152.92 75.278) (width 0.2) (layer "B.Cu") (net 5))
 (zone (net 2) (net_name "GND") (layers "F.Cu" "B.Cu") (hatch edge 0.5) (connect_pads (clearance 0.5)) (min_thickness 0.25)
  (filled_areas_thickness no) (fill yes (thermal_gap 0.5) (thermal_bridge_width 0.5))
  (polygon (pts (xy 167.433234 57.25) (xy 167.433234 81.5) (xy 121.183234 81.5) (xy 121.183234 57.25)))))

